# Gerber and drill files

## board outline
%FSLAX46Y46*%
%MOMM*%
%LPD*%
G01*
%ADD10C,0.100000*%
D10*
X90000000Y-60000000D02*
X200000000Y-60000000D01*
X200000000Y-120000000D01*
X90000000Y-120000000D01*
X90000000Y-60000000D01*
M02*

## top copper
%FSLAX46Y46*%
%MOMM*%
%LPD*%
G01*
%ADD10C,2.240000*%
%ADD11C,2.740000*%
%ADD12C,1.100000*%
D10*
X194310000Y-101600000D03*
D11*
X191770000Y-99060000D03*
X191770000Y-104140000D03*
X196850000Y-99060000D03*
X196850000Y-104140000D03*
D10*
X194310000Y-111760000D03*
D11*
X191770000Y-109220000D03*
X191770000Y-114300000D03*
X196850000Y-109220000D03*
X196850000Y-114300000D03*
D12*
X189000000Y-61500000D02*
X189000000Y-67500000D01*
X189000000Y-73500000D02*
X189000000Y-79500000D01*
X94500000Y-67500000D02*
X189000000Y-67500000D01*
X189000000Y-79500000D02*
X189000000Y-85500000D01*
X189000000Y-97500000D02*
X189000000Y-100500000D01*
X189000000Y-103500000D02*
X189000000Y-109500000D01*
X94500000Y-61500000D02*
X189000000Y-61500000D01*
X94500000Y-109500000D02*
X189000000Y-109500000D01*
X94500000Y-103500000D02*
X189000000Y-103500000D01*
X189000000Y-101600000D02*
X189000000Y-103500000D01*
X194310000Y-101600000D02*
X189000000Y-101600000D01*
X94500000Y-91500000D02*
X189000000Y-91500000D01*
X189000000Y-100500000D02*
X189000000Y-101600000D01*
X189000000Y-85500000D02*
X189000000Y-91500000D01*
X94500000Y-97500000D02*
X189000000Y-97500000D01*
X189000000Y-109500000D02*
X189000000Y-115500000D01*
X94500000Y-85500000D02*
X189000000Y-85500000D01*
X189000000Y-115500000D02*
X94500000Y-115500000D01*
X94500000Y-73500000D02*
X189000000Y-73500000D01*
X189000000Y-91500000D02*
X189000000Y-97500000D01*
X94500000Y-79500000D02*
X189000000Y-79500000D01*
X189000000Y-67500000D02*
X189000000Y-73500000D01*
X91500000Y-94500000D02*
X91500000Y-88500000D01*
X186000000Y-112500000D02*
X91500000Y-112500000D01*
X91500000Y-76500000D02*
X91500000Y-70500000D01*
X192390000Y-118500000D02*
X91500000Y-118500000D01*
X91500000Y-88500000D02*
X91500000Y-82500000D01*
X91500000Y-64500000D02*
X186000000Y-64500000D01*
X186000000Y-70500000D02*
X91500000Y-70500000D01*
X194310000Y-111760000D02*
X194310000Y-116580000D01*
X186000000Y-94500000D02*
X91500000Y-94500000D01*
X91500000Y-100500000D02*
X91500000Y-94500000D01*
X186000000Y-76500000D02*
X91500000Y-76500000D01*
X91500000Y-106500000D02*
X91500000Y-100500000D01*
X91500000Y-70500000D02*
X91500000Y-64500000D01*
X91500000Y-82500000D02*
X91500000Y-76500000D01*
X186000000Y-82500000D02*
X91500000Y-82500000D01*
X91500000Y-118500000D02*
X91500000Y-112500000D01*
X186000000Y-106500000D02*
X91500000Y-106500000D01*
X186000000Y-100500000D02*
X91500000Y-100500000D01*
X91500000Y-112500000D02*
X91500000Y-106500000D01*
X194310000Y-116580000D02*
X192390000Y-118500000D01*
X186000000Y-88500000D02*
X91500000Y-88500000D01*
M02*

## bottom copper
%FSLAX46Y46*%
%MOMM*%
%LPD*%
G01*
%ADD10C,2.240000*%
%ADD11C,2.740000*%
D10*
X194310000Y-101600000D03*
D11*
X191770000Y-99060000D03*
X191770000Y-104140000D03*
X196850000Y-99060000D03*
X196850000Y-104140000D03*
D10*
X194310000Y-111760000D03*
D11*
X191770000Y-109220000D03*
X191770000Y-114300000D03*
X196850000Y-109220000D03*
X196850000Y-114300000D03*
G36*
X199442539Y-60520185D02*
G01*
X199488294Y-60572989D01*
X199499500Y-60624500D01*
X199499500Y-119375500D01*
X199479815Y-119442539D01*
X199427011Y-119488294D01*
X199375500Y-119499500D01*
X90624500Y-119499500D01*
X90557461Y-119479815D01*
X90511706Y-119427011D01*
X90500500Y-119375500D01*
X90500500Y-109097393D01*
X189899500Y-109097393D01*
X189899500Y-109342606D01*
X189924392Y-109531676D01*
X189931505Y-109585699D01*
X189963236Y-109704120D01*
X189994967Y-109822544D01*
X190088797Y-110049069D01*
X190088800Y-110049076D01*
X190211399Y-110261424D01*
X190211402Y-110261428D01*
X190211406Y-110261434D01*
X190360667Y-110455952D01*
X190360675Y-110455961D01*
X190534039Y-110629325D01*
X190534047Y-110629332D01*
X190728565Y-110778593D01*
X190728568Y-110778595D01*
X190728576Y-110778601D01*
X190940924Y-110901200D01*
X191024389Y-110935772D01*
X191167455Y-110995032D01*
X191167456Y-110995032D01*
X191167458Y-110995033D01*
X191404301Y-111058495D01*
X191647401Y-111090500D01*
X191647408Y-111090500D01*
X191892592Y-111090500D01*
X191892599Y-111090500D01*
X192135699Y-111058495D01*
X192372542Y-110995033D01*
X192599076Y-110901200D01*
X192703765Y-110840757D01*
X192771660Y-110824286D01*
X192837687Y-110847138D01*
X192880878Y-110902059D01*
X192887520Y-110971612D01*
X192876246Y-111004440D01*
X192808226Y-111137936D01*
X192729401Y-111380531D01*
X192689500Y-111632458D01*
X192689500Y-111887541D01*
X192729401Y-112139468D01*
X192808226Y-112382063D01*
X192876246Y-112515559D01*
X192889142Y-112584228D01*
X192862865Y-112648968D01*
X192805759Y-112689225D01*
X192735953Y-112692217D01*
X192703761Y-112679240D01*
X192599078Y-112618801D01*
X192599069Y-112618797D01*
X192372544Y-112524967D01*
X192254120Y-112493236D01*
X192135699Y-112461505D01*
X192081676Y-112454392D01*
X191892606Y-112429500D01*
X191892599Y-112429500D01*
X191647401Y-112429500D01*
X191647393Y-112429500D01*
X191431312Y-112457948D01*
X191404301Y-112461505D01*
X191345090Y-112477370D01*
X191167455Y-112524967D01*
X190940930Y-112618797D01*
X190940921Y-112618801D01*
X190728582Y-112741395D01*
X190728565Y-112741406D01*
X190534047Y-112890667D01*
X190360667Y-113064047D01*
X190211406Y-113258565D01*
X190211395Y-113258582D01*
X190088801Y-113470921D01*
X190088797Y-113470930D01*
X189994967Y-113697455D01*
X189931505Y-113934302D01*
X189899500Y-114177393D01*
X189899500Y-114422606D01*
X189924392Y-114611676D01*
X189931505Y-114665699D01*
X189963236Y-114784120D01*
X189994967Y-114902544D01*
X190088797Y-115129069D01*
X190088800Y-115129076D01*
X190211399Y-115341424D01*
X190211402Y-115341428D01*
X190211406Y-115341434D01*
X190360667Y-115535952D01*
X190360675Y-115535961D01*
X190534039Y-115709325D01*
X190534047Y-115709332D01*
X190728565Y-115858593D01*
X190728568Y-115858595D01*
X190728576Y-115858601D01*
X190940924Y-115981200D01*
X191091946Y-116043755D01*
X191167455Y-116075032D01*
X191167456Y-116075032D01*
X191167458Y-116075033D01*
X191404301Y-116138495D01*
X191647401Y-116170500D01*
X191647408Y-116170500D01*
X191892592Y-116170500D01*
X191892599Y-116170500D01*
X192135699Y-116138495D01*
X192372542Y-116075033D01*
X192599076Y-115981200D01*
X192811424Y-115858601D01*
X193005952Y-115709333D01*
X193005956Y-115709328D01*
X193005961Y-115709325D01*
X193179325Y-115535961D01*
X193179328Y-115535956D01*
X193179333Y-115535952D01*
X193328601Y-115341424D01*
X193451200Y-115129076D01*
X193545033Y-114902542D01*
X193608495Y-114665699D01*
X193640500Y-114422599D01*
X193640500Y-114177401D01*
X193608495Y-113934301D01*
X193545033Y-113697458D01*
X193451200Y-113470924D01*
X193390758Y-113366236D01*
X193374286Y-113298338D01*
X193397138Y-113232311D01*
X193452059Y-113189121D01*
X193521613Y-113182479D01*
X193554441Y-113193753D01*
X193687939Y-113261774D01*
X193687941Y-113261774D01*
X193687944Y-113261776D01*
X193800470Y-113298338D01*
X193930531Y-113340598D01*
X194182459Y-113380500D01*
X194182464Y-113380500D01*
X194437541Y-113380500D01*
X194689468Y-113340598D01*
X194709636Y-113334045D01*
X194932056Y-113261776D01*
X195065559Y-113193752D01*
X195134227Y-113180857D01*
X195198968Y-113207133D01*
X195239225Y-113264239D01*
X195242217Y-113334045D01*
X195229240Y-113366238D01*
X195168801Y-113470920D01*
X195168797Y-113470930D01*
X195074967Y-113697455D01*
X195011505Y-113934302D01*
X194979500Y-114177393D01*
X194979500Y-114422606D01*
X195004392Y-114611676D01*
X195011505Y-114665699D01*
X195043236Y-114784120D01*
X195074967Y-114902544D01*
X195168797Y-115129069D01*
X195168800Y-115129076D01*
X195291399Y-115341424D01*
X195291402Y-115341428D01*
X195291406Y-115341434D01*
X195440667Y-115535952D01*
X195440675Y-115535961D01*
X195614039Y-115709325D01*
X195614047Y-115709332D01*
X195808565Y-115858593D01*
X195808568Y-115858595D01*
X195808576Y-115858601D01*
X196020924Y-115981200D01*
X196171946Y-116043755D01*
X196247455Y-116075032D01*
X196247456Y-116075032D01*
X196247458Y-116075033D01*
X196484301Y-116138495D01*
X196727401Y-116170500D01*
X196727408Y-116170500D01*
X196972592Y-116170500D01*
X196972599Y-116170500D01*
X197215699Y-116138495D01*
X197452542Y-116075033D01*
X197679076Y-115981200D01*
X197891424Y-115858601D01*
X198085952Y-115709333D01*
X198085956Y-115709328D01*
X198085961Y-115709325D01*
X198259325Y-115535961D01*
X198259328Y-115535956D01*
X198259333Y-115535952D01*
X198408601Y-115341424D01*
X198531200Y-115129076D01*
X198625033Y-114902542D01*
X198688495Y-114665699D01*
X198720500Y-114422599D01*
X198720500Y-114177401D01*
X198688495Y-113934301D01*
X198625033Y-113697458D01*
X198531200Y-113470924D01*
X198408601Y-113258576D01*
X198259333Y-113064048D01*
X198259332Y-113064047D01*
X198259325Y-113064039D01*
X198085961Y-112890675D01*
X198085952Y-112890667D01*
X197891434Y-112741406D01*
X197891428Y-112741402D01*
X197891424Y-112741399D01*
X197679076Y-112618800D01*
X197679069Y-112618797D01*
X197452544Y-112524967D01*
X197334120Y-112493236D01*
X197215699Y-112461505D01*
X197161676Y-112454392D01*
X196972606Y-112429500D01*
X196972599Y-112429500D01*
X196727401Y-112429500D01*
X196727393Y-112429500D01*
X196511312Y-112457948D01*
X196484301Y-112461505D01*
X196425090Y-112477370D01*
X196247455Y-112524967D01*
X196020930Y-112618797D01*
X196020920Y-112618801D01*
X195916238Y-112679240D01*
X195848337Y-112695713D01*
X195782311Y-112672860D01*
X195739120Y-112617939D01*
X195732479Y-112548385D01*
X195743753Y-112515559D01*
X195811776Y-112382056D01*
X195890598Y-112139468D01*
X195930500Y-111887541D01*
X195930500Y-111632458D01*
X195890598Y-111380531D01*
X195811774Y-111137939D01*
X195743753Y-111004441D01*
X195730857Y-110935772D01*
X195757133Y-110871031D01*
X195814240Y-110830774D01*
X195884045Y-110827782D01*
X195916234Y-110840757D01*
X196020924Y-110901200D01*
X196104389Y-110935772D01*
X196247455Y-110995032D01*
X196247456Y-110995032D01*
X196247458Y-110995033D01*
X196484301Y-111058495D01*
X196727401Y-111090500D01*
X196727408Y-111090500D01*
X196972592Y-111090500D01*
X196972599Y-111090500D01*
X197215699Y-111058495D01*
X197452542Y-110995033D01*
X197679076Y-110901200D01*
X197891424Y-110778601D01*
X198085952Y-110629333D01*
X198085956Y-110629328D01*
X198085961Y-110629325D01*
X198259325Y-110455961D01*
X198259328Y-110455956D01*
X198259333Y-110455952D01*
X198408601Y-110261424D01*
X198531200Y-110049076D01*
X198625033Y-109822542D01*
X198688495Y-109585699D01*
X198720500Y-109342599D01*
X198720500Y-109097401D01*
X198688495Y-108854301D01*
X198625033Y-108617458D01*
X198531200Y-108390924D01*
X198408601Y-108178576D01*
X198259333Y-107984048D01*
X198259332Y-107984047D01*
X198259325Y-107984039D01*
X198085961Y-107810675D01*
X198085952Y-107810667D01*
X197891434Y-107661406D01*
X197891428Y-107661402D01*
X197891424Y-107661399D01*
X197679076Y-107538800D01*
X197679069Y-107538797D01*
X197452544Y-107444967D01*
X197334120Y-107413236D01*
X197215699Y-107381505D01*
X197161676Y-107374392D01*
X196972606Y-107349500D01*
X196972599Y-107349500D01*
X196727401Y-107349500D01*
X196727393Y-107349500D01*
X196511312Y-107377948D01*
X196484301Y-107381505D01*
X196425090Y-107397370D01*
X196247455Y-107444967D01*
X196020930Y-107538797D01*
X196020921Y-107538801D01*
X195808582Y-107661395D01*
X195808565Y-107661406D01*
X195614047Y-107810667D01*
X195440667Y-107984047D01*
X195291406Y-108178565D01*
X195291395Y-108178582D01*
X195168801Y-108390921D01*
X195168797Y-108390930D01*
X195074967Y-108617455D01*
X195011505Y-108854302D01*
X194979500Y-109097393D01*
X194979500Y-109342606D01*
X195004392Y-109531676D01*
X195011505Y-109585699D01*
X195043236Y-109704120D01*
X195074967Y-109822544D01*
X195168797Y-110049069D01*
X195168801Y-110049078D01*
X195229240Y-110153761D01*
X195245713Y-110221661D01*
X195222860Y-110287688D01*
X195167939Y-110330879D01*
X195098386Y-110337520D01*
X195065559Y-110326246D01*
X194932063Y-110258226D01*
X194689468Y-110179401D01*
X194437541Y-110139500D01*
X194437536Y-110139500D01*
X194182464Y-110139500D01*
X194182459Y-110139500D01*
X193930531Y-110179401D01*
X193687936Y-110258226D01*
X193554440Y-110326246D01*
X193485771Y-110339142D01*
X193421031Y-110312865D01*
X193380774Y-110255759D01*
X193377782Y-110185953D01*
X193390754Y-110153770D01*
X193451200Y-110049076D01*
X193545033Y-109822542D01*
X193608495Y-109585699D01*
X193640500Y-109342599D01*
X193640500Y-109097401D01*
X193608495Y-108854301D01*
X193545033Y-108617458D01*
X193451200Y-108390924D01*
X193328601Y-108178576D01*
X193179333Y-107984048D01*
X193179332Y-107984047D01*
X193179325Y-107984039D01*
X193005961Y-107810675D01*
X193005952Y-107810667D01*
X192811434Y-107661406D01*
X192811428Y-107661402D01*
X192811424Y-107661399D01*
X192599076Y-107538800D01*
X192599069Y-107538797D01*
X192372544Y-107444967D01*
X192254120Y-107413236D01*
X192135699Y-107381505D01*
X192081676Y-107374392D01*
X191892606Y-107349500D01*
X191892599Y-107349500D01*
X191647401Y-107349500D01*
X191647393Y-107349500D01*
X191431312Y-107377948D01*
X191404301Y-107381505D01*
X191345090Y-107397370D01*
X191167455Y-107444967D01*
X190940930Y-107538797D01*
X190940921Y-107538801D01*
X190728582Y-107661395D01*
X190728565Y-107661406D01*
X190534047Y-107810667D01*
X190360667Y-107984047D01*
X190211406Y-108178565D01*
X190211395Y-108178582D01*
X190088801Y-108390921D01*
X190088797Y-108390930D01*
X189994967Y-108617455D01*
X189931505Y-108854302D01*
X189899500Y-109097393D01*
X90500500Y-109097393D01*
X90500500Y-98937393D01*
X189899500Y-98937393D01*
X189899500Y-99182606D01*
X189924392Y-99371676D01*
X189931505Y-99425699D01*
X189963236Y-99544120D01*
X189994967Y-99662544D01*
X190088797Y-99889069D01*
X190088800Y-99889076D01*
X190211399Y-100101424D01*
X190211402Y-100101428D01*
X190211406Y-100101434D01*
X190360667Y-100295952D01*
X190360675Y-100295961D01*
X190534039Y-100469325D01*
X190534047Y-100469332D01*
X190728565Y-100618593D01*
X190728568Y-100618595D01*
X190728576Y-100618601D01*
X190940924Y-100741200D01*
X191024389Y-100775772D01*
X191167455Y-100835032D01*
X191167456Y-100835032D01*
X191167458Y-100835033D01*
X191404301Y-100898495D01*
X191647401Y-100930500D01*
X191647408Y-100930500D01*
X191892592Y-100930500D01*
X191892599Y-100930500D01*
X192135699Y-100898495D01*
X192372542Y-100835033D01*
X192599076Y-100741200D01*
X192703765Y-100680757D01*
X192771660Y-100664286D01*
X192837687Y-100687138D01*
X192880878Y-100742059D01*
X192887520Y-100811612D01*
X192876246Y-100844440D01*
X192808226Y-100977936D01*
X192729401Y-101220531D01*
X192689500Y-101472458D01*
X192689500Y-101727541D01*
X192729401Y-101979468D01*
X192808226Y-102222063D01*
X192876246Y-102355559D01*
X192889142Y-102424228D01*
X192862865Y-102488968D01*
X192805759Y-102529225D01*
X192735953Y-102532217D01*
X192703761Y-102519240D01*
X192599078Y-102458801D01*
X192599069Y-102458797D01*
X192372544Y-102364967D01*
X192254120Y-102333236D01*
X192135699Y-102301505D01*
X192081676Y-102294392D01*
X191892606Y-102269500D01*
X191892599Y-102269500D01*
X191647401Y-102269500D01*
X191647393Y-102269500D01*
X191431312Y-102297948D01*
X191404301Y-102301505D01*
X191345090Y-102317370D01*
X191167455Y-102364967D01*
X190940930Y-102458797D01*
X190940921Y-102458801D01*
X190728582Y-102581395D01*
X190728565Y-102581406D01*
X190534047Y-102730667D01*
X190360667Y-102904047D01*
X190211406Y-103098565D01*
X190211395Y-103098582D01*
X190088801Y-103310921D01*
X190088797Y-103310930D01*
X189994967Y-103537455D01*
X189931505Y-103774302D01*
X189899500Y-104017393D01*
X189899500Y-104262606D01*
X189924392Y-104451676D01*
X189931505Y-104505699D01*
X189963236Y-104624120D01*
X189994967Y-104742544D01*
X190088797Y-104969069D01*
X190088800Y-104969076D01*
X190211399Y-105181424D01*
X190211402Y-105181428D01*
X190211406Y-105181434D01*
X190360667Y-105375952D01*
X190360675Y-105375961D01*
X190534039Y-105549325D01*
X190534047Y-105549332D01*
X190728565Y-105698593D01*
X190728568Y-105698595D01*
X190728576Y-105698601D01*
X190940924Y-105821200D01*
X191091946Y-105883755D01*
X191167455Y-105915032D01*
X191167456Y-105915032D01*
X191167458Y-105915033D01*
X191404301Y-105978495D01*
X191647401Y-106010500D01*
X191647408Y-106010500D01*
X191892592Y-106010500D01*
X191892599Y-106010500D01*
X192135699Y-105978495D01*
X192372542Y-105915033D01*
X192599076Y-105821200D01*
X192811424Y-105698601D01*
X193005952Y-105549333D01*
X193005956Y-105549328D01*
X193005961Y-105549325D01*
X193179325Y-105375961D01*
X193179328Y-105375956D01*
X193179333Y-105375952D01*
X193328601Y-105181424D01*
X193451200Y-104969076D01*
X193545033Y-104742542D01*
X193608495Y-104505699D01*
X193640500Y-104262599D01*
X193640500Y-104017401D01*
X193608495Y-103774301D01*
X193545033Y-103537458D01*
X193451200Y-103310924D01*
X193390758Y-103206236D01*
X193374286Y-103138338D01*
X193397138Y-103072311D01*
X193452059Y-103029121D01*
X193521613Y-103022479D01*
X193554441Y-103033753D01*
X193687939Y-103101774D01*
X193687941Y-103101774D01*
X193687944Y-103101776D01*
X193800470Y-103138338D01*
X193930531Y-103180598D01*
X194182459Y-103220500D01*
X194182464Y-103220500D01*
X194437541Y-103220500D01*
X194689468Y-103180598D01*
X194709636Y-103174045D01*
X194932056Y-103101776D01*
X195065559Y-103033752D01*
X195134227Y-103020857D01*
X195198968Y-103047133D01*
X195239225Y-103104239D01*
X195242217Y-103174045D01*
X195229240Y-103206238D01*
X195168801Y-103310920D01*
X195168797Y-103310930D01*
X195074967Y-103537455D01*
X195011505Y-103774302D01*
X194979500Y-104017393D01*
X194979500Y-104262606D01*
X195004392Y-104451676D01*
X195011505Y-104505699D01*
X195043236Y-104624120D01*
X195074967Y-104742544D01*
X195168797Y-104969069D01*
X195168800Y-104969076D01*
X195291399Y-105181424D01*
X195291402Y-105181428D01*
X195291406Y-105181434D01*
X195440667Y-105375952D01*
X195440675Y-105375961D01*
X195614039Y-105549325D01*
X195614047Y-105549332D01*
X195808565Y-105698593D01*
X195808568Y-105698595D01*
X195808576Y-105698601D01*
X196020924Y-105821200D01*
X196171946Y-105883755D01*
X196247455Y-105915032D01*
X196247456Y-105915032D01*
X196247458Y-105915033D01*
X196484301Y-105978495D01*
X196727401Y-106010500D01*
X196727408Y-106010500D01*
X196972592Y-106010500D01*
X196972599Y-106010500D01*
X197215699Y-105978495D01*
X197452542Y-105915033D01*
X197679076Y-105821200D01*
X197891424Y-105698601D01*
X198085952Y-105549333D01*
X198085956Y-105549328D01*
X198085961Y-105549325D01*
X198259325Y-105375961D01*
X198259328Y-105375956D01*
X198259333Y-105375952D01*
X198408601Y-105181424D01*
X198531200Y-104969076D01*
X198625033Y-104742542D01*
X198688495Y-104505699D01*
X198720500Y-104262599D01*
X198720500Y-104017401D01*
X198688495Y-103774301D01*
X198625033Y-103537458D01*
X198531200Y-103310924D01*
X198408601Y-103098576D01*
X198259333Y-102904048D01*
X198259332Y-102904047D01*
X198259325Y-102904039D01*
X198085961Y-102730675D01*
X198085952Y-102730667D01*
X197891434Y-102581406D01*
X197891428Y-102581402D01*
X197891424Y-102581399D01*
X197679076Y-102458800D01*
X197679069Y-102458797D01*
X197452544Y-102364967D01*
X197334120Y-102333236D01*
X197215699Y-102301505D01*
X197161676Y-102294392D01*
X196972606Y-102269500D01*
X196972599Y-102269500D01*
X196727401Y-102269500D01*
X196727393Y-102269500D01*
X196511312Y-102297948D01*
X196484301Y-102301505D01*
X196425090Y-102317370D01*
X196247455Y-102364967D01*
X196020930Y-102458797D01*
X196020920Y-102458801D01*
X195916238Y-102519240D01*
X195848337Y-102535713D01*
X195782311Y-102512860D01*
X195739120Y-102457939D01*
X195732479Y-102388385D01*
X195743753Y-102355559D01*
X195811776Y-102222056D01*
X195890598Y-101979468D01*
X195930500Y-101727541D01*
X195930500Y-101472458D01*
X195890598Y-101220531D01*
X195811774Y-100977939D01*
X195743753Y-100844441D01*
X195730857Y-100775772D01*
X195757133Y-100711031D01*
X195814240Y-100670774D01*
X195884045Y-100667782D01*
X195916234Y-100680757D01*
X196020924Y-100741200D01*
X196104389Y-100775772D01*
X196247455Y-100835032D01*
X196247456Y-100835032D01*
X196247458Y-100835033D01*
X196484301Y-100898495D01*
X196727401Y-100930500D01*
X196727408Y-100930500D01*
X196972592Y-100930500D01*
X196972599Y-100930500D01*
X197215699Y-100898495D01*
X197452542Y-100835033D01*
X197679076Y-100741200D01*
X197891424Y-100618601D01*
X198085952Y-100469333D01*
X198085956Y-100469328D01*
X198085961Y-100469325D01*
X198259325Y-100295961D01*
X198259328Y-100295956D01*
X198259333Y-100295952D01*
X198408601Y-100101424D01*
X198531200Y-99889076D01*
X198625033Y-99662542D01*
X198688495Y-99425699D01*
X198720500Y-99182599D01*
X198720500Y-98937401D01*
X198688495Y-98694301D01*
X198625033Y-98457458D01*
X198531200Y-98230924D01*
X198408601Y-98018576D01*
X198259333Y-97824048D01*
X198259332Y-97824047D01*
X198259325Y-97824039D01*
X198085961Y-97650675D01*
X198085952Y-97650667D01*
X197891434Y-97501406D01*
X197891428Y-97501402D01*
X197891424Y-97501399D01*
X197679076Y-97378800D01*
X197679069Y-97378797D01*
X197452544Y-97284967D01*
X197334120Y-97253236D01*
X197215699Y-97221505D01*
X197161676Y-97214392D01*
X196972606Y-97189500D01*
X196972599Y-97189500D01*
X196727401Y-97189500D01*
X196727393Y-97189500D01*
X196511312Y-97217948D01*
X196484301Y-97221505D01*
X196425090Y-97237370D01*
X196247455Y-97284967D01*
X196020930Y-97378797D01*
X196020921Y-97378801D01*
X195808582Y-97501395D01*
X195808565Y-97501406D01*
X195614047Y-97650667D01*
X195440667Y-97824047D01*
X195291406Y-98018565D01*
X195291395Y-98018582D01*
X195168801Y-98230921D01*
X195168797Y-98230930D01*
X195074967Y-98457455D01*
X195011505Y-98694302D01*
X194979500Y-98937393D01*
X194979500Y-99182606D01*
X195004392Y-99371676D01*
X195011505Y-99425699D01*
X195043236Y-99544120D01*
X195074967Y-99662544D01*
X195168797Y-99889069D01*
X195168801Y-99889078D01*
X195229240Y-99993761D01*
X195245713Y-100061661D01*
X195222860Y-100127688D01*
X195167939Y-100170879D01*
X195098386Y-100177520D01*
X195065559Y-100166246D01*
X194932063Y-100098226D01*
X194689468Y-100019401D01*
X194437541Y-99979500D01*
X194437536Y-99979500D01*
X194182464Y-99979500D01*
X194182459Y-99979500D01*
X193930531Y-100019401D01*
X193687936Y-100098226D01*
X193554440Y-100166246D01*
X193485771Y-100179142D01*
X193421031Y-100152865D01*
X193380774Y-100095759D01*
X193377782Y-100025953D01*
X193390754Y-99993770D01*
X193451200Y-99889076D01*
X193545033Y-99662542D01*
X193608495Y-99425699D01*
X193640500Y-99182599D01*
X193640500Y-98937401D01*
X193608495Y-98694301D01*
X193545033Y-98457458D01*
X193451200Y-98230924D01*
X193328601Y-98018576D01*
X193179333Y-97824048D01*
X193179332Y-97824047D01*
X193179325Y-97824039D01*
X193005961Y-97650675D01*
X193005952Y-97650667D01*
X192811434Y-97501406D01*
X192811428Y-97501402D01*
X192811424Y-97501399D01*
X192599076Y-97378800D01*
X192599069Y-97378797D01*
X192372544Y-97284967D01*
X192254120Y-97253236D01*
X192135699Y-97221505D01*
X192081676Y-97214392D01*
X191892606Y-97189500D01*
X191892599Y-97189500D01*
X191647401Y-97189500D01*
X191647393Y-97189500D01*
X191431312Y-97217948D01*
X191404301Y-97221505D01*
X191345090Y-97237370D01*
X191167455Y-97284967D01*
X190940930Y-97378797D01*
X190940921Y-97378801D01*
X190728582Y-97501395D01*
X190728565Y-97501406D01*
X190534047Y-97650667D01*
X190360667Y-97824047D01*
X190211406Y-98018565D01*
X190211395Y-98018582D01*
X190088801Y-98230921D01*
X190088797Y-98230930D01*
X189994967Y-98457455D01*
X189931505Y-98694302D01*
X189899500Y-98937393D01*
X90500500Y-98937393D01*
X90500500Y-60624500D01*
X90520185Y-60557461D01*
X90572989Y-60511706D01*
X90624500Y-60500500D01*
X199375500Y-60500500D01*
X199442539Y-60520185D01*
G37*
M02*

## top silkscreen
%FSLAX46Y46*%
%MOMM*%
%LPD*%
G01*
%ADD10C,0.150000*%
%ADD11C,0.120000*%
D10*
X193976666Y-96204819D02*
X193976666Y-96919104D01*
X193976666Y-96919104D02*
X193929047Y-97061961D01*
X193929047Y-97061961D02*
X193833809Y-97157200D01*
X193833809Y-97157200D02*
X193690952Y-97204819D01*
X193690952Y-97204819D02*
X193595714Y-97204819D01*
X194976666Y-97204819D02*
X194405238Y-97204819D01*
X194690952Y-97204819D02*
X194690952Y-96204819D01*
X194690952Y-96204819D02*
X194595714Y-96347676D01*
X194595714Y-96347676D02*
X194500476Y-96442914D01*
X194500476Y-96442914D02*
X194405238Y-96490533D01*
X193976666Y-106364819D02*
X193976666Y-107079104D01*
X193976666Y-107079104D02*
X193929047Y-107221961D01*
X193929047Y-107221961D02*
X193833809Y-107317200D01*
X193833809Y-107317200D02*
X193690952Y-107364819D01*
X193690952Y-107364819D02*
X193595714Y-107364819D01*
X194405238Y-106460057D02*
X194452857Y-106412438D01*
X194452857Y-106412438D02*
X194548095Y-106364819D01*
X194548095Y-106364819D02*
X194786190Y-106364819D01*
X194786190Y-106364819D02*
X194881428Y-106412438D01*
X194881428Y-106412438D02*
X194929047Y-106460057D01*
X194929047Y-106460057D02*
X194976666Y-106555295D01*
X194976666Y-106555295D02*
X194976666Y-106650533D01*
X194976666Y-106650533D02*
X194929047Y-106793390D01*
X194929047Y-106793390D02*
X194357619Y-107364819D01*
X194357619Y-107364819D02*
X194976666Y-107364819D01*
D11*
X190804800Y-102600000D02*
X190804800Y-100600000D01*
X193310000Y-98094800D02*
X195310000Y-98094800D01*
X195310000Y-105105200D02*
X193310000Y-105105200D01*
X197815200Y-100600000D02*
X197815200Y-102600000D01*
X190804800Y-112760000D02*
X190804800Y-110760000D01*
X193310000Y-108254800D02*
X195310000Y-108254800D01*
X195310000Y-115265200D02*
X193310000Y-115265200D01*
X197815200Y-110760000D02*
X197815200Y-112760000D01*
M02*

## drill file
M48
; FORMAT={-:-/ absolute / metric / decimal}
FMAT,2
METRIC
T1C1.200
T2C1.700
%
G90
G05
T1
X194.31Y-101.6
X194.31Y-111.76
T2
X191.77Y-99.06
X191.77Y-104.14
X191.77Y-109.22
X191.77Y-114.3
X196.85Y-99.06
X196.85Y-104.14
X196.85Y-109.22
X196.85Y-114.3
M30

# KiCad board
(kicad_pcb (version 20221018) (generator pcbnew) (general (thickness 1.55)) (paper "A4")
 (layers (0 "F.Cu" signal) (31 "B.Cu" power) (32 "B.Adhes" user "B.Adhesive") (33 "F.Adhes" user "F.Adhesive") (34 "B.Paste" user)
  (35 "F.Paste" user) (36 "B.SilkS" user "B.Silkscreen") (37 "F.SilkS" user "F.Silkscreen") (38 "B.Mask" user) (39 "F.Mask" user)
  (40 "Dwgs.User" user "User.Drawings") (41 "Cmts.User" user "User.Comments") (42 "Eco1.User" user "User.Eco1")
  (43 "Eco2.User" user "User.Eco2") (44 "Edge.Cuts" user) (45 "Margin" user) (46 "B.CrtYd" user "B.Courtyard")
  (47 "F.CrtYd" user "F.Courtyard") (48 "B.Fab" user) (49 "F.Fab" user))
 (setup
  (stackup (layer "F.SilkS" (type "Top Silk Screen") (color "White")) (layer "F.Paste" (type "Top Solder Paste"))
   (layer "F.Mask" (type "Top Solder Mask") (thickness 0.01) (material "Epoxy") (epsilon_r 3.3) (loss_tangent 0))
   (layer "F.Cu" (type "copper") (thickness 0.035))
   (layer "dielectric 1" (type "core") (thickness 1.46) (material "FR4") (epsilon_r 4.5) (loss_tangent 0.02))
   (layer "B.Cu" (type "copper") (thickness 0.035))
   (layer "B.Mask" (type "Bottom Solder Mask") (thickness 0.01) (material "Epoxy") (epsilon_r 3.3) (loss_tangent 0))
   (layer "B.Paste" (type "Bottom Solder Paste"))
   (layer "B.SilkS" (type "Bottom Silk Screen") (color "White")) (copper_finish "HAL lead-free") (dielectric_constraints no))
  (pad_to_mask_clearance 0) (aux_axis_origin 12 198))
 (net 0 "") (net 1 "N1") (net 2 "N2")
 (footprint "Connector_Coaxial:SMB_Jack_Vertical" (layer "F.Cu") (at 194.31 101.6)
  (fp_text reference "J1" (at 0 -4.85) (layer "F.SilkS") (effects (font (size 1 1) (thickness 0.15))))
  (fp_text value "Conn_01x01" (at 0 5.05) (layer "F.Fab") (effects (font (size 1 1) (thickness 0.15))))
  (fp_line (start -3.5052 1) (end -3.5052 -1) (stroke (width 0.12) (type solid)) (layer "F.SilkS"))
  (fp_line (start -1 -3.5052) (end 1 -3.5052) (stroke (width 0.12) (type solid)) (layer "F.SilkS"))
  (fp_line (start 1 3.5052) (end -1 3.5052) (stroke (width 0.12) (type solid)) (layer "F.SilkS"))
  (fp_line (start 3.5052 -1) (end 3.5052 1) (stroke (width 0.12) (type solid)) (layer "F.SilkS"))
  (pad "1" thru_hole circle (at 0 0) (size 2.24 2.24) (drill 1.2) (layers "*.Cu" "*.Mask") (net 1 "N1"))
  (pad "2" thru_hole circle (at -2.54 -2.54) (size 2.74 2.74) (drill 1.7) (layers "*.Cu" "*.Mask"))
  (pad "2" thru_hole circle (at -2.54 2.54) (size 2.74 2.74) (drill 1.7) (layers "*.Cu" "*.Mask"))
  (pad "2" thru_hole circle (at 2.54 -2.54) (size 2.74 2.74) (drill 1.7) (layers "*.Cu" "*.Mask"))
  (pad "2" thru_hole circle (at 2.54 2.54) (size 2.74 2.74) (drill 1.7) (layers "*.Cu" "*.Mask")))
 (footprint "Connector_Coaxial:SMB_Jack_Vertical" (layer "F.Cu") (at 194.31 111.76)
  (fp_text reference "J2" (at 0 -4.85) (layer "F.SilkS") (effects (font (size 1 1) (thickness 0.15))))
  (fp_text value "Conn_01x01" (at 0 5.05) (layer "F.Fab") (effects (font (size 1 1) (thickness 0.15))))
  (fp_line (start -3.5052 1) (end -3.5052 -1) (stroke (width 0.12) (type solid)) (layer "F.SilkS"))
  (fp_line (start -1 -3.5052) (end 1 -3.5052) (stroke (width 0.12) (type solid)) (layer "F.SilkS"))
  (fp_line (start 1 3.5052) (end -1 3.5052) (stroke (width 0.12) (type solid)) (layer "F.SilkS"))
  (fp_line (start 3.5052 -1) (end 3.5052 1) (stroke (width 0.12) (type solid)) (layer "F.SilkS"))
  (pad "1" thru_hole circle (at 0 0) (size 2.24 2.24) (drill 1.2) (layers "*.Cu" "*.Mask") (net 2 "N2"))
  (pad "2" thru_hole circle (at -2.54 -2.54) (size 2.74 2.74) (drill 1.7) (layers "*.Cu" "*.Mask"))
  (pad "2" thru_hole circle (at -2.54 2.54) (size 2.74 2.74) (drill 1.7) (layers "*.Cu" "*.Mask"))
  (pad "2" thru_hole circle (at 2.54 -2.54) (size 2.74 2.74) (drill 1.7) (layers "*.Cu" "*.Mask"))
  (pad "2" thru_hole circle (at 2.54 2.54) (size 2.74 2.74) (drill 1.7) (layers "*.Cu" "*.Mask")))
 (gr_rect (start 90 60) (end 200 120) (stroke (width 0.1) (type default)) (fill none) (layer "Edge.Cuts"))
 (segment (start 189 61.5) (end 189 67.5) (width 1.1) (layer "F.Cu") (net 1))
 (segment (start 189 73.5) (end 189 79.5) (width 1.1) (layer "F.Cu") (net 1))
 (segment (start 94.5 67.5) (end 189 67.5) (width 1.1) (layer "F.Cu") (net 1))
 (segment (start 189 79.5) (end 189 85.5) (width 1.1) (layer "F.Cu") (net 1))
 (segment (start 189 97.5) (end 189 100.5) (width 1.1) (layer "F.Cu") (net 1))
 (segment (start 189 103.5) (end 189 109.5) (width 1.1) (layer "F.Cu") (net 1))
 (segment (start 94.5 61.5) (end 189 61.5) (width 1.1) (layer "F.Cu") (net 1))
 (segment (start 94.5 109.5) (end 189 109.5) (width 1.1) (layer "F.Cu") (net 1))
 (segment (start 94.5 103.5) (end 189 103.5) (width 1.1) (layer "F.Cu") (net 1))
 (segment (start 189 101.6) (end 189 103.5) (width 1.1) (layer "F.Cu") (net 1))
 (segment (start 194.31 101.6) (end 189 101.6) (width 1.1) (layer "F.Cu") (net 1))
 (segment (start 94.5 91.5) (end 189 91.5) (width 1.1) (layer "F.Cu") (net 1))
 (segment (start 189 100.5) (end 189 101.6) (width 1.1) (layer "F.Cu") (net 1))
 (segment (start 189 85.5) (end 189 91.5) (width 1.1) (layer "F.Cu") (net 1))
 (segment (start 94.5 97.5) (end 189 97.5) (width 1.1) (layer "F.Cu") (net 1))
 (segment (start 189 109.5) (end 189 115.5) (width 1.1) (layer "F.Cu") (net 1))
 (segment (start 94.5 85.5) (end 189 85.5) (width 1.1) (layer "F.Cu") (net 1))
 (segment (start 189 115.5) (end 94.5 115.5) (width 1.1) (layer "F.Cu") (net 1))
 (segment (start 94.5 73.5) (end 189 73.5) (width 1.1) (layer "F.Cu") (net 1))
 (segment (start 189 91.5) (end 189 97.5) (width 1.1) (layer "F.Cu") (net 1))
 (segment (start 94.5 79.5) (end 189 79.5) (width 1.1) (layer "F.Cu") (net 1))
 (segment (start 189 67.5) (end 189 73.5) (width 1.1) (layer "F.Cu") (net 1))
 (segment (start 91.5 94.5) (end 91.5 88.5) (width 1.1) (layer "F.Cu") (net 2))
 (segment (start 186 112.5) (end 91.5 112.5) (width 1.1) (layer "F.Cu") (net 2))
 (segment (start 91.5 76.5) (end 91.5 70.5) (width 1.1) (layer "F.Cu") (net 2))
 (segment (start 192.39 118.5) (end 91.5 118.5) (width 1.1) (layer "F.Cu") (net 2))
 (segment (start 91.5 88.5) (end 91.5 82.5) (width 1.1) (layer "F.Cu") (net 2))
 (segment (start 91.5 64.5) (end 186 64.5) (width 1.1) (layer "F.Cu") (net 2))
 (segment (start 186 70.5) (end 91.5 70.5) (width 1.1) (layer "F.Cu") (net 2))
 (segment (start 194.31 111.76) (end 194.31 116.58) (width 1.1) (layer "F.Cu") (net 2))
 (segment (start 186 94.5) (end 91.5 94.5) (width 1.1) (layer "F.Cu") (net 2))
 (segment (start 91.5 100.5) (end 91.5 94.5) (width 1.1) (layer "F.Cu") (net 2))
 (segment (start 186 76.5) (end 91.5 76.5) (width 1.1) (layer "F.Cu") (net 2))
 (segment (start 91.5 106.5) (end 91.5 100.5) (width 1.1) (layer "F.Cu") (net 2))
 (segment (start 91.5 70.5) (end 91.5 64.5) (width 1.1) (layer "F.Cu") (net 2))
 (segment (start 91.5 82.5) (end 91.5 76.5) (width 1.1) (layer "F.Cu") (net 2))
 (segment (start 186 82.5) (end 91.5 82.5) (width 1.1) (layer "F.Cu") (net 2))
 (segment (start 91.5 118.5) (end 91.5 112.5) (width 1.1) (layer "F.Cu") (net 2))
 (segment (start 186 106.5) (end 91.5 106.5) (width 1.1) (layer "F.Cu") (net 2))
 (segment (start 186 100.5) (end 91.5 100.5) (width 1.1) (layer "F.Cu") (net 2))
 (segment (start 91.5 112.5) (end 91.5 106.5) (width 1.1) (layer "F.Cu") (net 2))
 (segment (start 194.31 116.58) (end 192.39 118.5) (width 1.1) (layer "F.Cu") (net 2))
 (segment (start 186 88.5) (end 91.5 88.5) (width 1.1) (layer "F.Cu") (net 2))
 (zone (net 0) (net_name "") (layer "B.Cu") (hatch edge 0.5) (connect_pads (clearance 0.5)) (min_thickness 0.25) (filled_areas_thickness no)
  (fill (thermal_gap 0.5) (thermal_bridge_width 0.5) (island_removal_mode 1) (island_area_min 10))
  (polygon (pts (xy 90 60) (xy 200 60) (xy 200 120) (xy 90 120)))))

